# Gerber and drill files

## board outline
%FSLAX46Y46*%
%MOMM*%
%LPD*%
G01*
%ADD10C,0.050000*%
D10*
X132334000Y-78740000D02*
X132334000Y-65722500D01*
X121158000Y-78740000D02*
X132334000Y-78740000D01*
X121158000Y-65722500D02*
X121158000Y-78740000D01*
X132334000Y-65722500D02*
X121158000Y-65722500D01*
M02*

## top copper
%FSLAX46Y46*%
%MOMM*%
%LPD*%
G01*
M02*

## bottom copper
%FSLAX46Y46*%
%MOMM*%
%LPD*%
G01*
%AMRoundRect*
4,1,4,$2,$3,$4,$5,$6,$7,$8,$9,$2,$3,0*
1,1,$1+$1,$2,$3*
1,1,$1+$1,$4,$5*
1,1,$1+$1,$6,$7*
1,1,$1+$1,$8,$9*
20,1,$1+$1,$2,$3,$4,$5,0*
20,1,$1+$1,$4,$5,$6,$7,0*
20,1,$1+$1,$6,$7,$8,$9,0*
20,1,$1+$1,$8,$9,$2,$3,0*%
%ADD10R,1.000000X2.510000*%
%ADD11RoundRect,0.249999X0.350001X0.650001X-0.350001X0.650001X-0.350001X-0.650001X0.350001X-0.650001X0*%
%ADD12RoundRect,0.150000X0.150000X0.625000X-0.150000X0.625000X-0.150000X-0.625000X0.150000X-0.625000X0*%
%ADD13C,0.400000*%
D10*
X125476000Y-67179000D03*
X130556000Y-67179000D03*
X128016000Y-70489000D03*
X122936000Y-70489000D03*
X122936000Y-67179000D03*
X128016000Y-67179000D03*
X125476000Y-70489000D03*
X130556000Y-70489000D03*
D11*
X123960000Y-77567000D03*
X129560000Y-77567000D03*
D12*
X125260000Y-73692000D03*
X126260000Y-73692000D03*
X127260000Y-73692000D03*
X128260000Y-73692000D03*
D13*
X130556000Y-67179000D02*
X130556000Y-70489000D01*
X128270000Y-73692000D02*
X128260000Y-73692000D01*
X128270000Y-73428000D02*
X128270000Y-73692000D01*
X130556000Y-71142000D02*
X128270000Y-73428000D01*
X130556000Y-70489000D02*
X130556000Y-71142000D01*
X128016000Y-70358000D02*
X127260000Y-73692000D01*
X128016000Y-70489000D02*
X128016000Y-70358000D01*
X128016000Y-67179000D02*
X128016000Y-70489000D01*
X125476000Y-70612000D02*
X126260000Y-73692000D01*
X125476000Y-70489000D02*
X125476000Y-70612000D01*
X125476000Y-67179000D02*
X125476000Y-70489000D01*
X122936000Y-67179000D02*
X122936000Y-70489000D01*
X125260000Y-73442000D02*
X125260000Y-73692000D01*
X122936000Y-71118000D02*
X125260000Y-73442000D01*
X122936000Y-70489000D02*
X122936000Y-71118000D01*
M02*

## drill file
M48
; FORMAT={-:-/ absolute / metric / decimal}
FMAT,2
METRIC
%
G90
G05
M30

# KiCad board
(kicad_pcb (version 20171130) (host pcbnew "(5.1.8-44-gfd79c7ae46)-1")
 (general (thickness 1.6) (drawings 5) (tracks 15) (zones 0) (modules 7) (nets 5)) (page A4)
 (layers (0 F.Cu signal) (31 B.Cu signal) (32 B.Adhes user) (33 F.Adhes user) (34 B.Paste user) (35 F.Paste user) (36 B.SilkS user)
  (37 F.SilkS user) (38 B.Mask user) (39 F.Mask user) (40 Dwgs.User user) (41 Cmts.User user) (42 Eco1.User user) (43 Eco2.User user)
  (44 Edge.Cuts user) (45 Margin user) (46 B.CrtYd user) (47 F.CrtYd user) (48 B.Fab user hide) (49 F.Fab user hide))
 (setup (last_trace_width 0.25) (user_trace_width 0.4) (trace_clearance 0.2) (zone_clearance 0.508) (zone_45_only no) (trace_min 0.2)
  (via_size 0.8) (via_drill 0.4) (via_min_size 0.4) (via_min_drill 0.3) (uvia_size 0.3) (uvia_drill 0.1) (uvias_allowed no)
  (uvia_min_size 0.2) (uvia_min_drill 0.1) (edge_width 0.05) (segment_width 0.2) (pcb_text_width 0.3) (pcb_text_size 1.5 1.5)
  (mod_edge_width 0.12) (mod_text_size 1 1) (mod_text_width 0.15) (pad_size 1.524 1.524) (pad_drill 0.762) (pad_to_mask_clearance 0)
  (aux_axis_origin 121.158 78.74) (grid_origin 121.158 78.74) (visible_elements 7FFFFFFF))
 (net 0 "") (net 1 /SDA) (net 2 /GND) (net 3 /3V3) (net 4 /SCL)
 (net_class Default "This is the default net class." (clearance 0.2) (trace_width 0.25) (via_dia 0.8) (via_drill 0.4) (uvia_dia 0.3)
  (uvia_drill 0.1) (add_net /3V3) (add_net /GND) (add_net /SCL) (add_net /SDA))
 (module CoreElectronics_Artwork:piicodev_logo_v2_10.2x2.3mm (layer F.Cu) (at 126.770646 72.644)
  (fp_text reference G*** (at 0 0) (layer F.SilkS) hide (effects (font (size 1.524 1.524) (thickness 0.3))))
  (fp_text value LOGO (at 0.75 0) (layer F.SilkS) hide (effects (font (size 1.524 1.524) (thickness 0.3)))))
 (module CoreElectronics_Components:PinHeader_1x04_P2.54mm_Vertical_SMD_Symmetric (layer B.Cu) (at 126.746 68.834 90)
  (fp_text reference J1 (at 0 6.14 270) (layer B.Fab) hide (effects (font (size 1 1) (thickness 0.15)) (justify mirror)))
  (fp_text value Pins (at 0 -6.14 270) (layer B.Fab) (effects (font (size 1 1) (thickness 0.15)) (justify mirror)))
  (pad 3 smd rect (at 1.655 -1.27 90) (size 2.51 1) (layers B.Cu B.Paste B.Mask) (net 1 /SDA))
  (pad 1 smd rect (at 1.655 3.81 90) (size 2.51 1) (layers B.Cu B.Paste B.Mask) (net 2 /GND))
  (pad 2 smd rect (at -1.655 1.27 90) (size 2.51 1) (layers B.Cu B.Paste B.Mask) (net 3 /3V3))
  (pad 4 smd rect (at -1.655 -3.81 90) (size 2.51 1) (layers B.Cu B.Paste B.Mask) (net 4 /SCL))
  (pad 4 smd rect (at 1.655 -3.81 90) (size 2.51 1) (layers B.Cu B.Paste B.Mask) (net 4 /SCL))
  (pad 2 smd rect (at 1.655 1.27 90) (size 2.51 1) (layers B.Cu B.Paste B.Mask) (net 3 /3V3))
  (pad 3 smd rect (at -1.655 -1.27 90) (size 2.51 1) (layers B.Cu B.Paste B.Mask) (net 1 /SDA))
  (pad 1 smd rect (at -1.655 3.81 90) (size 2.51 1) (layers B.Cu B.Paste B.Mask) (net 2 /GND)))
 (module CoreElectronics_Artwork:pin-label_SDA (layer F.Cu) (at 125.476 68.326 270)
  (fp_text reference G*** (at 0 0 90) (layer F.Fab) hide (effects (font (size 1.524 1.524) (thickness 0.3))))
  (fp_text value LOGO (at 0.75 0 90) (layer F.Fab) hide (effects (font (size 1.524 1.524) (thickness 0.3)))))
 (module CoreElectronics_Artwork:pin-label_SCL (layer F.Cu) (at 122.936 68.326 270)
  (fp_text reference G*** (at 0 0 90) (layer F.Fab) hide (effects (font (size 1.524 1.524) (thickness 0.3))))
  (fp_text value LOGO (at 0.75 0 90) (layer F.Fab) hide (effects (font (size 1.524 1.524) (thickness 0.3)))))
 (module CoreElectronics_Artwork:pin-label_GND (layer F.Cu) (at 130.556 68.326 270)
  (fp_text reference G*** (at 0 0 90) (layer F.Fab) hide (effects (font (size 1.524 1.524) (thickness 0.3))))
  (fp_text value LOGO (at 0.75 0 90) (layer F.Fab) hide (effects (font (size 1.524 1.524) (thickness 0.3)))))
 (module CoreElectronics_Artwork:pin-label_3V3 (layer F.Cu) (at 128.016 68.326 270)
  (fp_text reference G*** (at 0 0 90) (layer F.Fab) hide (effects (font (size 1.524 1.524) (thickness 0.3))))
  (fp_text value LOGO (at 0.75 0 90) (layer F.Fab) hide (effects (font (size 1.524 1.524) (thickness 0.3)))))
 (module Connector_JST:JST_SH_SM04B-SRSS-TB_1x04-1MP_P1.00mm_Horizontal (layer B.Cu) (at 126.76 75.692 180)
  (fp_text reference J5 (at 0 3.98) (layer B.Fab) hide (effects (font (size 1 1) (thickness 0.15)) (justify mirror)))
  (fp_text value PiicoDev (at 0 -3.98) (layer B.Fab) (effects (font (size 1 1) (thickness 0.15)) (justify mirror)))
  (pad MP smd roundrect (at 2.8 -1.875 180) (size 1.2 1.8) (layers B.Cu B.Paste B.Mask) (roundrect_rratio 0.2083325))
  (pad MP smd roundrect (at -2.8 -1.875 180) (size 1.2 1.8) (layers B.Cu B.Paste B.Mask) (roundrect_rratio 0.2083325))
  (pad 4 smd roundrect (at 1.5 2 180) (size 0.6 1.55) (layers B.Cu B.Paste B.Mask) (roundrect_rratio 0.25) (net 4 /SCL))
  (pad 3 smd roundrect (at 0.5 2 180) (size 0.6 1.55) (layers B.Cu B.Paste B.Mask) (roundrect_rratio 0.25) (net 1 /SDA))
  (pad 2 smd roundrect (at -0.5 2 180) (size 0.6 1.55) (layers B.Cu B.Paste B.Mask) (roundrect_rratio 0.25) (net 3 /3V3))
  (pad 1 smd roundrect (at -1.5 2 180) (size 0.6 1.55) (layers B.Cu B.Paste B.Mask) (roundrect_rratio 0.25) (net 2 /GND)))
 (gr_line (start 132.334 78.74) (end 132.334 65.7225) (layer Edge.Cuts) (width 0.05))
 (gr_line (start 121.158 78.74) (end 132.334 78.74) (layer Edge.Cuts) (width 0.05))
 (gr_line (start 121.158 65.7225) (end 121.158 78.74) (layer Edge.Cuts) (width 0.05))
 (gr_line (start 132.334 65.7225) (end 121.158 65.7225) (layer Edge.Cuts) (width 0.05))
 (segment (start 130.556 67.179) (end 130.556 70.489) (width 0.4) (layer B.Cu) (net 2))
 (segment (start 128.27 73.692) (end 128.26 73.692) (width 0.4) (layer B.Cu) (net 2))
 (segment (start 128.27 73.428) (end 128.27 73.692) (width 0.4) (layer B.Cu) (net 2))
 (segment (start 130.556 71.142) (end 128.27 73.428) (width 0.4) (layer B.Cu) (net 2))
 (segment (start 130.556 70.489) (end 130.556 71.142) (width 0.4) (layer B.Cu) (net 2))
 (segment (start 128.016 70.358) (end 127.26 73.692) (width 0.4) (layer B.Cu) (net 3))
 (segment (start 128.016 70.489) (end 128.016 70.358) (width 0.4) (layer B.Cu) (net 3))
 (segment (start 128.016 67.179) (end 128.016 70.489) (width 0.4) (layer B.Cu) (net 3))
 (segment (start 125.476 70.612) (end 126.26 73.692) (width 0.4) (layer B.Cu) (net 1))
 (segment (start 125.476 70.489) (end 125.476 70.612) (width 0.4) (layer B.Cu) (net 1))
 (segment (start 125.476 67.179) (end 125.476 70.489) (width 0.4) (layer B.Cu) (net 1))
 (segment (start 122.936 67.179) (end 122.936 70.489) (width 0.4) (layer B.Cu) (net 4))
 (segment (start 125.26 73.442) (end 125.26 73.692) (width 0.4) (layer B.Cu) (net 4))
 (segment (start 122.936 71.118) (end 125.26 73.442) (width 0.4) (layer B.Cu) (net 4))
 (segment (start 122.936 70.489) (end 122.936 71.118) (width 0.4) (layer B.Cu) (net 4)))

